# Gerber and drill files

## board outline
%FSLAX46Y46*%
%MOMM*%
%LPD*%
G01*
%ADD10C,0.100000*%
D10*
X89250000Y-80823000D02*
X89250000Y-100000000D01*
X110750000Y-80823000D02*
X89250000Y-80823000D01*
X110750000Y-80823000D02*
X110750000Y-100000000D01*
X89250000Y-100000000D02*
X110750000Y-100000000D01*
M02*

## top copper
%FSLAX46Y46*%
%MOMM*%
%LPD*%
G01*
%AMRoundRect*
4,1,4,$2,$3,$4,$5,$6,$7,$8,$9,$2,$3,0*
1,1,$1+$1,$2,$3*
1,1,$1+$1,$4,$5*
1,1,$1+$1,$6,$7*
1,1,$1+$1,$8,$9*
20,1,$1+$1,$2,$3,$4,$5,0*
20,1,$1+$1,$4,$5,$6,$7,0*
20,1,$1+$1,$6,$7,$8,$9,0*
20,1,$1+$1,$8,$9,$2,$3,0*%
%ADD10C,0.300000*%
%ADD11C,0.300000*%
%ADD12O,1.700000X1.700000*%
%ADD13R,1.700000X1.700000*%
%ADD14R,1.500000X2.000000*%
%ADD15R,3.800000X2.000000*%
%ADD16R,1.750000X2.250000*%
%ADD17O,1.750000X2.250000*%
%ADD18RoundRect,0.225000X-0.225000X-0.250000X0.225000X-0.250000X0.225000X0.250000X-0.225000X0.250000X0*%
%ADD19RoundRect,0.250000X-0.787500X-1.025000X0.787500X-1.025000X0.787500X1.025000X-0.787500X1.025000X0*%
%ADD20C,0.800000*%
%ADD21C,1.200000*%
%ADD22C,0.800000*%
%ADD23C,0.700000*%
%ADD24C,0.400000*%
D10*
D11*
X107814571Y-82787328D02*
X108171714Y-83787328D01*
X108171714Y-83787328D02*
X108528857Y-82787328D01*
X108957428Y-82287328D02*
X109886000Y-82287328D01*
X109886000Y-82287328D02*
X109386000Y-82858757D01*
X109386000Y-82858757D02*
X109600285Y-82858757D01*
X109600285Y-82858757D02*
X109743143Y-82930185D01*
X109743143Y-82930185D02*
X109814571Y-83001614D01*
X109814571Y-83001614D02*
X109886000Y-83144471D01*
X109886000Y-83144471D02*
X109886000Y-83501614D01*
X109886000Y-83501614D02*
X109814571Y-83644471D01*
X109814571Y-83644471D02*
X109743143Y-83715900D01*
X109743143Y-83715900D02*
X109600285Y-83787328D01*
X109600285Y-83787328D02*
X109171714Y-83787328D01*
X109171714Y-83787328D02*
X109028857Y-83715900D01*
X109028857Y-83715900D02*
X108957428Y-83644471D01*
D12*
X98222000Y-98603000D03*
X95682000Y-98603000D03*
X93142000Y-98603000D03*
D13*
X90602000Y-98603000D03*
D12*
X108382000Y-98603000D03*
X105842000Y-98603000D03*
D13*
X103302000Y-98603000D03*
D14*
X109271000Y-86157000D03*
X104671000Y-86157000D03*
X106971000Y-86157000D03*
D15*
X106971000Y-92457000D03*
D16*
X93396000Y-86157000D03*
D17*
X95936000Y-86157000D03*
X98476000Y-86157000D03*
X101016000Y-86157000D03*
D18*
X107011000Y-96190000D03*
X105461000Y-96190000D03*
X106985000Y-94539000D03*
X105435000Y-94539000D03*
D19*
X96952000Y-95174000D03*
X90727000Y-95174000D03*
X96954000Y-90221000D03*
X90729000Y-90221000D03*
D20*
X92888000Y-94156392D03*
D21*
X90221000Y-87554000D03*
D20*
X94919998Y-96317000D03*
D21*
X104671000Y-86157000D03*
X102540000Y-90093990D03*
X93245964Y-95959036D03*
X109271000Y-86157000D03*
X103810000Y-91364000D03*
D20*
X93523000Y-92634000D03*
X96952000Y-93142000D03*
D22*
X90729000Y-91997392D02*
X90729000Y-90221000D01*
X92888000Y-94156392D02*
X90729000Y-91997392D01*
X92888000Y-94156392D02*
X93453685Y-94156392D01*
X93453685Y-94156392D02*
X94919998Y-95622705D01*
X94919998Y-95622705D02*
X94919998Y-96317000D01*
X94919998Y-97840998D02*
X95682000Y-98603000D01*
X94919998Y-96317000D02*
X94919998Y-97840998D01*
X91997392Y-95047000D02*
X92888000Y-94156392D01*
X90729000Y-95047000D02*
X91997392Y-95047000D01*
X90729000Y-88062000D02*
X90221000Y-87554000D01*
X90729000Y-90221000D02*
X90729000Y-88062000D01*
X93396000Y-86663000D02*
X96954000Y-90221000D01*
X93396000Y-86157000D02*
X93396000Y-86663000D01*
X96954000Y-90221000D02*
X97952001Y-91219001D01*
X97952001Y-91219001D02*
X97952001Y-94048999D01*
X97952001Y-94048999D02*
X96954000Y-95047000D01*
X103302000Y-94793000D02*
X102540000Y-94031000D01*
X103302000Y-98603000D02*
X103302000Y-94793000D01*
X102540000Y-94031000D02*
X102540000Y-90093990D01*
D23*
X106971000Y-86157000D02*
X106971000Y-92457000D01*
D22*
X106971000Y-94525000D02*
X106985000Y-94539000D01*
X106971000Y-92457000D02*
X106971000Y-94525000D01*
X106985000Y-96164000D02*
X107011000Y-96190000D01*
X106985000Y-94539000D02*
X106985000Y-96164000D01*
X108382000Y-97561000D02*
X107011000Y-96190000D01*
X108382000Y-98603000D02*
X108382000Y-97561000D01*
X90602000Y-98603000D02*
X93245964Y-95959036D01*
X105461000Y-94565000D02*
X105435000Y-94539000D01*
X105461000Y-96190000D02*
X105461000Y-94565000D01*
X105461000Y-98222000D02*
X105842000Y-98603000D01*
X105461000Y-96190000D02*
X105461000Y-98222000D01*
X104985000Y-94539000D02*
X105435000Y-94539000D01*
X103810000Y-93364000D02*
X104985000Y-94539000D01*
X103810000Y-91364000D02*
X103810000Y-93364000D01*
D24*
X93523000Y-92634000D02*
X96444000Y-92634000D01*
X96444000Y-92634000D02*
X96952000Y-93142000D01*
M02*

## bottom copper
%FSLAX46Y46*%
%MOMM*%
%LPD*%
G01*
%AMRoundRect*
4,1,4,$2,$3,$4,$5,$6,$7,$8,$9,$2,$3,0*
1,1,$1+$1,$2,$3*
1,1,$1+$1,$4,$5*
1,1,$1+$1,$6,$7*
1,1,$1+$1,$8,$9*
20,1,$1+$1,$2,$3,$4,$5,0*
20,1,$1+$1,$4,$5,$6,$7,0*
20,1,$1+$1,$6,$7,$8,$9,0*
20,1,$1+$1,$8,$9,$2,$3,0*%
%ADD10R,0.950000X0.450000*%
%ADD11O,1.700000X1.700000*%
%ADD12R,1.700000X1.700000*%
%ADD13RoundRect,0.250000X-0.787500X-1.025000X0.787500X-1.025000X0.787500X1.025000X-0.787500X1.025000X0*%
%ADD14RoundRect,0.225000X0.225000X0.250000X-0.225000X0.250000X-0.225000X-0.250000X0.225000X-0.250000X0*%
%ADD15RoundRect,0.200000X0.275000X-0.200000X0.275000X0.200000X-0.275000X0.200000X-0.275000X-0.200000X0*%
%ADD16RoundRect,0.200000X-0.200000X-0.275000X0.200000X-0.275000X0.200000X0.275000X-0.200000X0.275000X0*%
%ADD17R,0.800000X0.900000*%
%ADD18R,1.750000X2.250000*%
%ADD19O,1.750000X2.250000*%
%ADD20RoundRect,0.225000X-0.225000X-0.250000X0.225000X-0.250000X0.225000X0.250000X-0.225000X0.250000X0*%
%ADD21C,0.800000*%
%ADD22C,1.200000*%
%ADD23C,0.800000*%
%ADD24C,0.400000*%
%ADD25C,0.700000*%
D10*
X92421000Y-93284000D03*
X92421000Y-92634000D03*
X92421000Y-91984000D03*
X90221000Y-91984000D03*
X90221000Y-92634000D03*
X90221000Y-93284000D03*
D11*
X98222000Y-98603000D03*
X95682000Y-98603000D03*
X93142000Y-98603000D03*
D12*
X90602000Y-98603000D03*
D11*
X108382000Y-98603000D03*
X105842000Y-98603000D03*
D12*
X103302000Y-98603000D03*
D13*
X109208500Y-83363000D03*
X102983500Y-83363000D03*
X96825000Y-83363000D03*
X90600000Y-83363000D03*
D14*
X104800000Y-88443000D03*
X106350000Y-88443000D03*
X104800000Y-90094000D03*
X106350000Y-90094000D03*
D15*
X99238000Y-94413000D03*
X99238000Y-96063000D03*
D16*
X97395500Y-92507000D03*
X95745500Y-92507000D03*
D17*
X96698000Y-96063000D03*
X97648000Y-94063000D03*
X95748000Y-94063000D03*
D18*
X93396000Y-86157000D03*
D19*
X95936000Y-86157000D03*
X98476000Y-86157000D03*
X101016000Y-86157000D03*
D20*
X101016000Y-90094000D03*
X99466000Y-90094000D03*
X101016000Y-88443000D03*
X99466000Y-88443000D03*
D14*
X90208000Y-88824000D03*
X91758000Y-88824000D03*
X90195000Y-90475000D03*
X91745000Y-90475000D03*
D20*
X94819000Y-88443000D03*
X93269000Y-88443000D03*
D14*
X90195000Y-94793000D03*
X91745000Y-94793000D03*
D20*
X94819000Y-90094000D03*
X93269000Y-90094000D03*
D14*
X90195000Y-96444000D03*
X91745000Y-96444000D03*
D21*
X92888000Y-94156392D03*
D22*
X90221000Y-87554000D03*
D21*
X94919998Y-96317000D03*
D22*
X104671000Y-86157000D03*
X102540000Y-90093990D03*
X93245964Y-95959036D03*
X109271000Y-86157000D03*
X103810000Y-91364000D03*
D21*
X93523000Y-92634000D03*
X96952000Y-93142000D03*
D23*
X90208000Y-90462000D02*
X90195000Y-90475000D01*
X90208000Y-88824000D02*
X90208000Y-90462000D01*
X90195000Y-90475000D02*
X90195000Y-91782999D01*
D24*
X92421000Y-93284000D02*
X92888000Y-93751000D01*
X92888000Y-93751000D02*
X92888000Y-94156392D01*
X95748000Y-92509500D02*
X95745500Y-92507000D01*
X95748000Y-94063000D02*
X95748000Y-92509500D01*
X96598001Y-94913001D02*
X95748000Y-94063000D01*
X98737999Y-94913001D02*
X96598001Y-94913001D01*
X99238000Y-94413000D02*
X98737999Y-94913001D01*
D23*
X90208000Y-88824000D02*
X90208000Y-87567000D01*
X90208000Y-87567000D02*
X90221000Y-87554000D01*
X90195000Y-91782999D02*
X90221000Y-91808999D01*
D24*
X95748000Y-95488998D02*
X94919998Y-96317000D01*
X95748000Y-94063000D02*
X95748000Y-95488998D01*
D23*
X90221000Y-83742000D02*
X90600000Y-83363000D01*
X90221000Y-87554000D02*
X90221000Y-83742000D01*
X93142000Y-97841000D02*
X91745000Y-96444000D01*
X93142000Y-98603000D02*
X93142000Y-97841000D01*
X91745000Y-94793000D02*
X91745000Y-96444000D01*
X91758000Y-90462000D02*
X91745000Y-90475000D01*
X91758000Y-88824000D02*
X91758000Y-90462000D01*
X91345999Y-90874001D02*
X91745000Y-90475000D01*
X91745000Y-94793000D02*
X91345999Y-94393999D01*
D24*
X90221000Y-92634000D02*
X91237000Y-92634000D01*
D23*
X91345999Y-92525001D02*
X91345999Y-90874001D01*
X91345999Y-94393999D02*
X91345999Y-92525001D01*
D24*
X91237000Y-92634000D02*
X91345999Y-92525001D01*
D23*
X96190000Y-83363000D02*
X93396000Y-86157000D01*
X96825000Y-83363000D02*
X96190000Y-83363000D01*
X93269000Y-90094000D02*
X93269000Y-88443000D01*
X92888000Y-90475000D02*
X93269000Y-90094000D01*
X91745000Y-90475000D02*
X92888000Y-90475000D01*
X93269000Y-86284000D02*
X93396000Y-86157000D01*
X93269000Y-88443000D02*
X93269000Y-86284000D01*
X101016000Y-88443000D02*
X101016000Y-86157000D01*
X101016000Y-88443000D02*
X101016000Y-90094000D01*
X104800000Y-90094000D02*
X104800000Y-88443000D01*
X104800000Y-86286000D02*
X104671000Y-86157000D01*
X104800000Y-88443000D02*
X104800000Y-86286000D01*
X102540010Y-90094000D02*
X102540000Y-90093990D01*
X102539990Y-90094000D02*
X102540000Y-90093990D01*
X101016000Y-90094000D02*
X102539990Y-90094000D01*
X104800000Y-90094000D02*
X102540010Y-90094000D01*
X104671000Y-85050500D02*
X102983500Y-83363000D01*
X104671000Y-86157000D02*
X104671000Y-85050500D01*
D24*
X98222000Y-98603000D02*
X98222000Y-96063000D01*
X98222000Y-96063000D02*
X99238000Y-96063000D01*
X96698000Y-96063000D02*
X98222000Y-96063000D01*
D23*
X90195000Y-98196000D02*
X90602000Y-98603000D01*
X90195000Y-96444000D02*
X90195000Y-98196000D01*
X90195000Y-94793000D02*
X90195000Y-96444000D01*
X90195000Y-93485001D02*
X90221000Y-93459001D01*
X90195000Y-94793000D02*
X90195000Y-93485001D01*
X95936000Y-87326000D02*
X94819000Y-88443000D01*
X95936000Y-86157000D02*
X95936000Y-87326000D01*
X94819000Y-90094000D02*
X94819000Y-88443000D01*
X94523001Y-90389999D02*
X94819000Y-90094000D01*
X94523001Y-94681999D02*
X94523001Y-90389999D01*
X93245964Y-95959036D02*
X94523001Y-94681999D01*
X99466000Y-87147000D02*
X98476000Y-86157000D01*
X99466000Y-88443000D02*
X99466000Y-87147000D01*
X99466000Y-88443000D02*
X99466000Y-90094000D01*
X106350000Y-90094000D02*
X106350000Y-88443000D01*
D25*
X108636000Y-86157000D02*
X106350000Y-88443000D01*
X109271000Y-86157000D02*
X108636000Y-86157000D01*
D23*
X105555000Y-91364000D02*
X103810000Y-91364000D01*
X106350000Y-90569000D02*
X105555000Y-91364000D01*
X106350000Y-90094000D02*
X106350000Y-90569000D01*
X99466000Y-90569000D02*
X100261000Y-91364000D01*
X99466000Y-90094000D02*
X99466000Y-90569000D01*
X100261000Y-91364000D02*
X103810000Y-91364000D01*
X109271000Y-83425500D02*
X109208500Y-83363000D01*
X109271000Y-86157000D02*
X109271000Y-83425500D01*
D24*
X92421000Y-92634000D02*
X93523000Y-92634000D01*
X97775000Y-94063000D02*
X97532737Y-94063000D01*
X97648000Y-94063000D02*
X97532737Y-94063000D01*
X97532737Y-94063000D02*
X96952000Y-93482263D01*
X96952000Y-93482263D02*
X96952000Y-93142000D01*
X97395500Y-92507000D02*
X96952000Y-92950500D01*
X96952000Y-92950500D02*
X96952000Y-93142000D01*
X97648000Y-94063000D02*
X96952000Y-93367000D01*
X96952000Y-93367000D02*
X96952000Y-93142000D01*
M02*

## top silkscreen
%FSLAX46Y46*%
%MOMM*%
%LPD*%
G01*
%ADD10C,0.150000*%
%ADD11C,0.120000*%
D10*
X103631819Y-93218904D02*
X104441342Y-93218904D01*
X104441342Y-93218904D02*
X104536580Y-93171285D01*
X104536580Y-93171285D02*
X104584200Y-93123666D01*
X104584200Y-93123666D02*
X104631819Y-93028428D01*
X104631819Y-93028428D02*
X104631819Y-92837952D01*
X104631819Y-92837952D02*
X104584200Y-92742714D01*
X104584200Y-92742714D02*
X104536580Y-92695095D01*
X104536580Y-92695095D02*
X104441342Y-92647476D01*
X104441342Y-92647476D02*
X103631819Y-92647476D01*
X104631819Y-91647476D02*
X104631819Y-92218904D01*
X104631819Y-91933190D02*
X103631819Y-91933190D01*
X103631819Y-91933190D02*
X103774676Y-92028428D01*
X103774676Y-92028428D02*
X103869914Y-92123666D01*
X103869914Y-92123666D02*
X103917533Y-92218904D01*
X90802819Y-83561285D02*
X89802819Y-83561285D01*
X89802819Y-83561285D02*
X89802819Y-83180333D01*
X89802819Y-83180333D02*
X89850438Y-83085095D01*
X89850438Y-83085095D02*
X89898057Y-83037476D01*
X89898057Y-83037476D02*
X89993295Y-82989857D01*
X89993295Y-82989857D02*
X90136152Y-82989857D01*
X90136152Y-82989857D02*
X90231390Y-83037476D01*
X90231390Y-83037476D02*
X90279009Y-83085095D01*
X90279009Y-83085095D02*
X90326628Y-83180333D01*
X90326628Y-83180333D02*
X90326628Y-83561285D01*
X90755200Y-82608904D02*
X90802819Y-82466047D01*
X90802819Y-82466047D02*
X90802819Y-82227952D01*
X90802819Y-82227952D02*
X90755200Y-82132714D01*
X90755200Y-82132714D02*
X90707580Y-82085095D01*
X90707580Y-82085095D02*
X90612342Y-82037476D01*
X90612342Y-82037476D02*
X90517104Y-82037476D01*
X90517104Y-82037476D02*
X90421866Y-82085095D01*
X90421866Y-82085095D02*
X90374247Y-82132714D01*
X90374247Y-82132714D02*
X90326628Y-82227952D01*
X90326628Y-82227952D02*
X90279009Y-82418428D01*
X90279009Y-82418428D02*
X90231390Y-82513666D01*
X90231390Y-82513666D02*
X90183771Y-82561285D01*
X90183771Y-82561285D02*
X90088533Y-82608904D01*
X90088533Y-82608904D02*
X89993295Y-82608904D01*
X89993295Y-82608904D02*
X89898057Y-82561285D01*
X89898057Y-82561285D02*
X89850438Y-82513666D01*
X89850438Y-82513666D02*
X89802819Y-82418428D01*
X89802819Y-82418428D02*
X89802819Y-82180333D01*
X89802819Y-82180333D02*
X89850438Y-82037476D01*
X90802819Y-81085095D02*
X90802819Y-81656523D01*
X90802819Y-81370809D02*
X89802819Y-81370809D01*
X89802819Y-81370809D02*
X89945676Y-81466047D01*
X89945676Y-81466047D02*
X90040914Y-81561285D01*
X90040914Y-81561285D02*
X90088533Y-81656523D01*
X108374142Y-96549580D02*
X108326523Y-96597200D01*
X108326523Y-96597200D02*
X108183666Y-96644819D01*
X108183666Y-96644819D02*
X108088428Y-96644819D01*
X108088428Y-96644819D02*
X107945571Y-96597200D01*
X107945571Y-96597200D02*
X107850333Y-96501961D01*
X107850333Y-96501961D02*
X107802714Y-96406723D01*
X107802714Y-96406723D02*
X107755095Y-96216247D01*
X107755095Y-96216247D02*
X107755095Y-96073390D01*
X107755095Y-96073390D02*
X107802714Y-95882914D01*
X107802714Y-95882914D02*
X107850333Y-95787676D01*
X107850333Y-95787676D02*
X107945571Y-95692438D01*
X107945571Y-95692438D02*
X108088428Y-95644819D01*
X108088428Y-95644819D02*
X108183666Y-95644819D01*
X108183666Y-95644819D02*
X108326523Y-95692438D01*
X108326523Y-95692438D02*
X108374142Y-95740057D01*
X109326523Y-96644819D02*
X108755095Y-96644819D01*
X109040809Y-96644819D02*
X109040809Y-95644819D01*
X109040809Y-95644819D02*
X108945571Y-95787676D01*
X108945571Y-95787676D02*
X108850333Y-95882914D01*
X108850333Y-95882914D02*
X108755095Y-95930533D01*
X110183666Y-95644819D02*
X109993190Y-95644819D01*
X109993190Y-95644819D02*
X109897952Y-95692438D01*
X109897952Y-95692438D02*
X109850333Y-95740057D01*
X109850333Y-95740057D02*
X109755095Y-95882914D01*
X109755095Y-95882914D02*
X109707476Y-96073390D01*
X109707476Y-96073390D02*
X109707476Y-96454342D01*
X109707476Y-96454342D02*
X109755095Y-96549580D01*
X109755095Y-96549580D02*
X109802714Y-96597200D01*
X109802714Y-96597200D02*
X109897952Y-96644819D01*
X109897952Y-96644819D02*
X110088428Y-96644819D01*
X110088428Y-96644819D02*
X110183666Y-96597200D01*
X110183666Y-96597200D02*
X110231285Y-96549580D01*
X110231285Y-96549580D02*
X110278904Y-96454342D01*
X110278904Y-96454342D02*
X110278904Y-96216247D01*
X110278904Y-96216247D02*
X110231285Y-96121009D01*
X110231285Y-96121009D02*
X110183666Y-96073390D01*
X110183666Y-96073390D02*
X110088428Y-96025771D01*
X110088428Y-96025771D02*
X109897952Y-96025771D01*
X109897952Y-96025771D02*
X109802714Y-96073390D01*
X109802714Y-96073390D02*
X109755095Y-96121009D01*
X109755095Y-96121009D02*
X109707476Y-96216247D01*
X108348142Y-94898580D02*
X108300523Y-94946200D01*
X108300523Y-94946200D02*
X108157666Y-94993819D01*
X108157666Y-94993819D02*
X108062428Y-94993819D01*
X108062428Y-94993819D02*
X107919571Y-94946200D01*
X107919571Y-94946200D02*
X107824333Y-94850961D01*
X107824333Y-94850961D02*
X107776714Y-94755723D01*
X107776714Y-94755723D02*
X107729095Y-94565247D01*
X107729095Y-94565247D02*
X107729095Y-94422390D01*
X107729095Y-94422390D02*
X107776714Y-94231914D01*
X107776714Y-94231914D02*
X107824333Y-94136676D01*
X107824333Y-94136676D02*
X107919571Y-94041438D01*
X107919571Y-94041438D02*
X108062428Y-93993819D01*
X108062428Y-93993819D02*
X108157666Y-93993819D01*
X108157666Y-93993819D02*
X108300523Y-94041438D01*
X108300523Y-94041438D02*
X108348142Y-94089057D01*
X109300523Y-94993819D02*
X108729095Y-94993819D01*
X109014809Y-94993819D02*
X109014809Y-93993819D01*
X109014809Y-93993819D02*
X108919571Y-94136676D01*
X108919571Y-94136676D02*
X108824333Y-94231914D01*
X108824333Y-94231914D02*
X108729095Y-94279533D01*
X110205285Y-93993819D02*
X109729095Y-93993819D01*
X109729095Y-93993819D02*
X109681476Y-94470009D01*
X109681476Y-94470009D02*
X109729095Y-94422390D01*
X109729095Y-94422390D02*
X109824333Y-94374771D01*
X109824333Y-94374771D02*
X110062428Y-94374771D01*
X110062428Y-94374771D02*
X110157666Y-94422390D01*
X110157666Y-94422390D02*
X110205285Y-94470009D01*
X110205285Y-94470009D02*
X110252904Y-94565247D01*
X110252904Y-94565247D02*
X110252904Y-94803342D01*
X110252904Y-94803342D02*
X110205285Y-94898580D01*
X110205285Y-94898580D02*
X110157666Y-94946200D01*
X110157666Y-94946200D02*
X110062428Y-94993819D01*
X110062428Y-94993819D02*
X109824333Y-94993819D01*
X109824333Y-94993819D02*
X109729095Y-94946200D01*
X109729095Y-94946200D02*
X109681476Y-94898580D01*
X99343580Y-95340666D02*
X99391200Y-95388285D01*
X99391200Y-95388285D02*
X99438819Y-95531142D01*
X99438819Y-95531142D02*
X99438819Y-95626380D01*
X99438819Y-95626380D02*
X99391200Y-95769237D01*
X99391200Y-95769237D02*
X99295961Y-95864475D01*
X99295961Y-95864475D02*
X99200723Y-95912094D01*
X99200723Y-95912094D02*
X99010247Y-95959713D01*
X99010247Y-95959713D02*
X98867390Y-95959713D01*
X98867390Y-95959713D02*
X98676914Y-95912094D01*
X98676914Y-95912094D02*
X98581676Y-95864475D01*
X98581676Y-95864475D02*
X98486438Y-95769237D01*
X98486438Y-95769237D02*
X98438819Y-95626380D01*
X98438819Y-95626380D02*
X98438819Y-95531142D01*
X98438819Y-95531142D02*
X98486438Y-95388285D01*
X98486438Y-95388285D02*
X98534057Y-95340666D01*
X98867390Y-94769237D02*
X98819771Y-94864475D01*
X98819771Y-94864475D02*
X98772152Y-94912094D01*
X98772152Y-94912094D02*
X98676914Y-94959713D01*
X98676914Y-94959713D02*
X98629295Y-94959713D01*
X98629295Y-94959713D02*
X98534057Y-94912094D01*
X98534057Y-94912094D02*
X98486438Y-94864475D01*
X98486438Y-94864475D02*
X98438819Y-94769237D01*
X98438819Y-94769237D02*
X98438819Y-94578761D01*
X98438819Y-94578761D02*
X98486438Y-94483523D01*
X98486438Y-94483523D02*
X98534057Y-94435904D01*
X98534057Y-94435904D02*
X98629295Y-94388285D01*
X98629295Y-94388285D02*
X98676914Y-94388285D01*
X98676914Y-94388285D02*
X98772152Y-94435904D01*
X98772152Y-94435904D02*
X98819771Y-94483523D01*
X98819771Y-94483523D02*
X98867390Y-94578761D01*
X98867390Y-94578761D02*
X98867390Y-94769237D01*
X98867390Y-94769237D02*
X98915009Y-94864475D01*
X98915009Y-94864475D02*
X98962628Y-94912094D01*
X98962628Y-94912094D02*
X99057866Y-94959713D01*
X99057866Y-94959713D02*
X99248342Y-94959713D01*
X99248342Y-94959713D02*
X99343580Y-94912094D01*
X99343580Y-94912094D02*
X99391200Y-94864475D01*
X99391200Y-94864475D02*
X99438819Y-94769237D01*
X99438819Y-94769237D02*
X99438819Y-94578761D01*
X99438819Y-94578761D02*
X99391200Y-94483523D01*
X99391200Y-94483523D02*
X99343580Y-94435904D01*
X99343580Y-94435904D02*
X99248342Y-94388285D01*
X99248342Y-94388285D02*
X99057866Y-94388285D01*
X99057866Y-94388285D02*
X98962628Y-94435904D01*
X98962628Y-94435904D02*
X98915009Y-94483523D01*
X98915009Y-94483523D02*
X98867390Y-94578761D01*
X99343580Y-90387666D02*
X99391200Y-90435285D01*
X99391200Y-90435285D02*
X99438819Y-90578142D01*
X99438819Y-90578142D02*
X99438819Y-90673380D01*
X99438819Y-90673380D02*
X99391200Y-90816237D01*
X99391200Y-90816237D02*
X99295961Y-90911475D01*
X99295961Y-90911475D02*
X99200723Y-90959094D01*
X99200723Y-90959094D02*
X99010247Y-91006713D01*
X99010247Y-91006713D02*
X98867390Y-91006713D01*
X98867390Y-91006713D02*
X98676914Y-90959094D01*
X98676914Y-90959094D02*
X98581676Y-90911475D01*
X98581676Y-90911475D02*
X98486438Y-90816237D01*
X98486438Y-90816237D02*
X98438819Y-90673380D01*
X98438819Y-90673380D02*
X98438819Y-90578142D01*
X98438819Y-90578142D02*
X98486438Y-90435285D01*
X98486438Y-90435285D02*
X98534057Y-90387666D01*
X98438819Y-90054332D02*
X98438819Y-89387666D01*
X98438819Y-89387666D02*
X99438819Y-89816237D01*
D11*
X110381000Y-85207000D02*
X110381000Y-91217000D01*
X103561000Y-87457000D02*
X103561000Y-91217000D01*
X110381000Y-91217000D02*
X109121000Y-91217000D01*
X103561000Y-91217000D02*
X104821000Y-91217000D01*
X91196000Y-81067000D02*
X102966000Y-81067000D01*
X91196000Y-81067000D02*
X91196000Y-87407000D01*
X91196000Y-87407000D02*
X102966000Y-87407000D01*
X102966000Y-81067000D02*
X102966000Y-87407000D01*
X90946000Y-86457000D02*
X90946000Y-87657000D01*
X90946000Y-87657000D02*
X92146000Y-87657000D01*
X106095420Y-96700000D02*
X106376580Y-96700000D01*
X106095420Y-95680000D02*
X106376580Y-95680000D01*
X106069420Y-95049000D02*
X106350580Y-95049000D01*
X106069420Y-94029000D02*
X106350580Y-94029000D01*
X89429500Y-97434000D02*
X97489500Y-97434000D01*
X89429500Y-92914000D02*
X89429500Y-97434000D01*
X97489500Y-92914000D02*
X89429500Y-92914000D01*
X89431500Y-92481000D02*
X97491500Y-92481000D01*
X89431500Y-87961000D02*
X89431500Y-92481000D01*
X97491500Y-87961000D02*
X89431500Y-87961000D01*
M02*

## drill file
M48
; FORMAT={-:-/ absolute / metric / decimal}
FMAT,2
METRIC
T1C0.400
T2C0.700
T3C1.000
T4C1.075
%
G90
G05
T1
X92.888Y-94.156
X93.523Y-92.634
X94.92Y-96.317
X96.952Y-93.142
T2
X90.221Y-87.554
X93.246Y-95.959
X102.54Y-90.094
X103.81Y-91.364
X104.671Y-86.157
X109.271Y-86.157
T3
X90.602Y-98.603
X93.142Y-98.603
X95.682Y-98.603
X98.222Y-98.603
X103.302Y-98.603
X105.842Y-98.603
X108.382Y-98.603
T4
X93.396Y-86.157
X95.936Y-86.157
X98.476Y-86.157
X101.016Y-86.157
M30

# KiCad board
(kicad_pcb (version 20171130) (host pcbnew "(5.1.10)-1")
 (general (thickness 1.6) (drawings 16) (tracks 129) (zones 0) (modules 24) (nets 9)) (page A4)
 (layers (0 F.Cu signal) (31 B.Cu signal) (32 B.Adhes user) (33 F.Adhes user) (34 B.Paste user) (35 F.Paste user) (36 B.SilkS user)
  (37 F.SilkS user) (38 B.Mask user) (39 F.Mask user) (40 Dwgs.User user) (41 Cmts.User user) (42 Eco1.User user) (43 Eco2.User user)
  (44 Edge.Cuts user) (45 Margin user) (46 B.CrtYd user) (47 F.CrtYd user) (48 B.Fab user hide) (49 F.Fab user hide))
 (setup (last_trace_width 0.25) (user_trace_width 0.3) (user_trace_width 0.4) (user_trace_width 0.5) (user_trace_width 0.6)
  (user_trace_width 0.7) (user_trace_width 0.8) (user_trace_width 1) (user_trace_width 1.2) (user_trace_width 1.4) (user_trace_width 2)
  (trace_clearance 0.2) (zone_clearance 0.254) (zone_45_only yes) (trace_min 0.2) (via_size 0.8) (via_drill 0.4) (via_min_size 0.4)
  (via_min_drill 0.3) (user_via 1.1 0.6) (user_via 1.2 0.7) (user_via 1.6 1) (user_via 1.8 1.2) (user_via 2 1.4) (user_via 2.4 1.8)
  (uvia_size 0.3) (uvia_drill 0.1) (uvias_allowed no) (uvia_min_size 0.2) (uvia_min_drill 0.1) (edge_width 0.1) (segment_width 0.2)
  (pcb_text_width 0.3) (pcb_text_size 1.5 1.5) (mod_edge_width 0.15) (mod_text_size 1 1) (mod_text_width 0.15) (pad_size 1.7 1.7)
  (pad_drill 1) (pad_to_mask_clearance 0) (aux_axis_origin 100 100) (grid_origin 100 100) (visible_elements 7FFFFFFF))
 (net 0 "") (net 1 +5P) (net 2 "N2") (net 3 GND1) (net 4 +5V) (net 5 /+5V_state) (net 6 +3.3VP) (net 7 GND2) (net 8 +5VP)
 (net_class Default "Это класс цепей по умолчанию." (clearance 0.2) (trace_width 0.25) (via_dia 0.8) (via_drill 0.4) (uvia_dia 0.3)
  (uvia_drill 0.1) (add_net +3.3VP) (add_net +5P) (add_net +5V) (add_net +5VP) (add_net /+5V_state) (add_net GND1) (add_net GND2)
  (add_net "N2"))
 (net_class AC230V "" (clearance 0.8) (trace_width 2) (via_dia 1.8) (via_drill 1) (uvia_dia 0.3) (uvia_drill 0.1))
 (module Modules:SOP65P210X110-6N (layer B.Cu) (at 91.321 92.634)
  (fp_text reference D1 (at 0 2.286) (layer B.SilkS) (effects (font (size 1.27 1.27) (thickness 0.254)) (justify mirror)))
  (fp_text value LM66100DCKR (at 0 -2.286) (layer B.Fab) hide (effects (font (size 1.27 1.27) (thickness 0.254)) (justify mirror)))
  (pad 6 smd rect (at 1.1 0.65 270) (size 0.45 0.95) (layers B.Cu B.Paste B.Mask) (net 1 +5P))
  (pad 5 smd rect (at 1.1 0 270) (size 0.45 0.95) (layers B.Cu B.Paste B.Mask) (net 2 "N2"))
  (pad 4 smd rect (at 1.1 -0.65 270) (size 0.45 0.95) (layers B.Cu B.Paste B.Mask))
  (pad 3 smd rect (at -1.1 -0.65 270) (size 0.45 0.95) (layers B.Cu B.Paste B.Mask) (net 1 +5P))
  (pad 2 smd rect (at -1.1 0 270) (size 0.45 0.95) (layers B.Cu B.Paste B.Mask) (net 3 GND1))
  (pad 1 smd rect (at -1.1 0.65 270) (size 0.45 0.95) (layers B.Cu B.Paste B.Mask) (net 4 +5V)))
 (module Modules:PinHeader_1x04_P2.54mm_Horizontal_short (layer B.Cu) (at 90.602 98.603 270)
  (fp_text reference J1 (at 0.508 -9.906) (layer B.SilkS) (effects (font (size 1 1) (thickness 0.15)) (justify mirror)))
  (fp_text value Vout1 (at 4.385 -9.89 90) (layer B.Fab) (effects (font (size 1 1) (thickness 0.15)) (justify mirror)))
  (pad 4 thru_hole oval (at 0 -7.62 270) (size 1.7 1.7) (drill 1) (layers *.Cu *.Mask) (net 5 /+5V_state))
  (pad 3 thru_hole oval (at 0 -5.08 270) (size 1.7 1.7) (drill 1) (layers *.Cu *.Mask) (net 1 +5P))
  (pad 2 thru_hole oval (at 0 -2.54 270) (size 1.7 1.7) (drill 1) (layers *.Cu *.Mask) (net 3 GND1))
  (pad 1 thru_hole rect (at 0 0 270) (size 1.7 1.7) (drill 1) (layers *.Cu *.Mask) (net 4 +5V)))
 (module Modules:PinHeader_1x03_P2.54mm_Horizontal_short (layer B.Cu) (at 103.302 98.603 270)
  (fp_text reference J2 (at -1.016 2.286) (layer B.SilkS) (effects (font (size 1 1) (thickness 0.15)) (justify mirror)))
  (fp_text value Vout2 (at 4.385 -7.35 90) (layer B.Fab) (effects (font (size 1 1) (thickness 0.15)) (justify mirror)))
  (pad 3 thru_hole oval (at 0 -5.08 270) (size 1.7 1.7) (drill 1) (layers *.Cu *.Mask) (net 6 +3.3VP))
  (pad 2 thru_hole oval (at 0 -2.54 270) (size 1.7 1.7) (drill 1) (layers *.Cu *.Mask) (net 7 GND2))
  (pad 1 thru_hole rect (at 0 0 270) (size 1.7 1.7) (drill 1) (layers *.Cu *.Mask) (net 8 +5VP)))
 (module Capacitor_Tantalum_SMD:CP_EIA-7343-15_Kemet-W (layer B.Cu) (at 106.096 83.363)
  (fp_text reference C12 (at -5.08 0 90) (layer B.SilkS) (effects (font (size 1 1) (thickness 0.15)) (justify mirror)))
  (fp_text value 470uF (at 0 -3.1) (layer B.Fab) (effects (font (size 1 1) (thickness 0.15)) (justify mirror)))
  (pad 2 smd roundrect (at 3.1125 0) (size 2.075 2.55) (layers B.Cu B.Paste B.Mask) (roundrect_rratio 0.1204819277108434) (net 7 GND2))
  (pad 1 smd roundrect (at -3.1125 0) (size 2.075 2.55) (layers B.Cu B.Paste B.Mask) (roundrect_rratio 0.1204819277108434) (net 8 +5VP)))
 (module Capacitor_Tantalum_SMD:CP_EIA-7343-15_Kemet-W (layer B.Cu) (at 93.7125 83.363)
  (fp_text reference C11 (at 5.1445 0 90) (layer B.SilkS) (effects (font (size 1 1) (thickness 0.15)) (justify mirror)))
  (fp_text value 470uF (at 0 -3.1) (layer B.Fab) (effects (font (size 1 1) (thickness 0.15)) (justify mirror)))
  (pad 2 smd roundrect (at 3.1125 0) (size 2.075 2.55) (layers B.Cu B.Paste B.Mask) (roundrect_rratio 0.1204819277108434) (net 3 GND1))
  (pad 1 smd roundrect (at -3.1125 0) (size 2.075 2.55) (layers B.Cu B.Paste B.Mask) (roundrect_rratio 0.1204819277108434) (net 1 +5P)))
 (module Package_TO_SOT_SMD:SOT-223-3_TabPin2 (layer F.Cu) (at 106.971 89.307 270)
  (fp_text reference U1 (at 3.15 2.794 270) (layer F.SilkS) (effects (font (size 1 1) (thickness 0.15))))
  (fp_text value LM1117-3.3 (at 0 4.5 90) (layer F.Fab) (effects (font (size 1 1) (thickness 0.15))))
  (fp_line (start -4.1 -3.41) (end 1.91 -3.41) (layer F.SilkS) (width 0.12))
  (fp_line (start -1.85 3.41) (end 1.91 3.41) (layer F.SilkS) (width 0.12))
  (fp_line (start 1.91 -3.41) (end 1.91 -2.15) (layer F.SilkS) (width 0.12))
  (fp_line (start 1.91 3.41) (end 1.91 2.15) (layer F.SilkS) (width 0.12))
  (pad 1 smd rect (at -3.15 -2.3 270) (size 2 1.5) (layers F.Cu F.Paste F.Mask) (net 7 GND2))
  (pad 3 smd rect (at -3.15 2.3 270) (size 2 1.5) (layers F.Cu F.Paste F.Mask) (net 8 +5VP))
  (pad 2 smd rect (at -3.15 0 270) (size 2 1.5) (layers F.Cu F.Paste F.Mask) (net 6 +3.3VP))
  (pad 2 smd rect (at 3.15 0 270) (size 2 3.8) (layers F.Cu F.Paste F.Mask) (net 6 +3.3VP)))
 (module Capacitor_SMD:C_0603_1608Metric (layer B.Cu) (at 105.575 88.443 180)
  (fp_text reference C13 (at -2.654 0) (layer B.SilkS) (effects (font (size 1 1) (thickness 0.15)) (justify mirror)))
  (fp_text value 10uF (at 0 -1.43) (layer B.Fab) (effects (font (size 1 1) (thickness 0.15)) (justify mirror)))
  (pad 2 smd roundrect (at 0.775 0 180) (size 0.9 0.95) (layers B.Cu B.Paste B.Mask) (roundrect_rratio 0.25) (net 8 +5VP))
  (pad 1 smd roundrect (at -0.775 0 180) (size 0.9 0.95) (layers B.Cu B.Paste B.Mask) (roundrect_rratio 0.25) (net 7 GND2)))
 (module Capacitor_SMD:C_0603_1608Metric (layer B.Cu) (at 105.575 90.094 180)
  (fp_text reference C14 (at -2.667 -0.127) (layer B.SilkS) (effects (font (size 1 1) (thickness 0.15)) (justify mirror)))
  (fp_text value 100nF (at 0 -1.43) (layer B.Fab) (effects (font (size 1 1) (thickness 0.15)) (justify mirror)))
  (pad 2 smd roundrect (at 0.775 0 180) (size 0.9 0.95) (layers B.Cu B.Paste B.Mask) (roundrect_rratio 0.25) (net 8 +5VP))
  (pad 1 smd roundrect (at -0.775 0 180) (size 0.9 0.95) (layers B.Cu B.Paste B.Mask) (roundrect_rratio 0.25) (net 7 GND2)))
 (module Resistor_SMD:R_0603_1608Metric (layer B.Cu) (at 99.238 95.238 90)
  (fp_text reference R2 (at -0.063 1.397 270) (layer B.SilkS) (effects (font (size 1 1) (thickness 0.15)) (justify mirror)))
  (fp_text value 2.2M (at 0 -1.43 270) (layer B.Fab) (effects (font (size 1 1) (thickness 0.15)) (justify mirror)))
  (pad 2 smd roundrect (at 0.825 0 90) (size 0.8 0.95) (layers B.Cu B.Paste B.Mask) (roundrect_rratio 0.25) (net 1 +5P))
  (pad 1 smd roundrect (at -0.825 0 90) (size 0.8 0.95) (layers B.Cu B.Paste B.Mask) (roundrect_rratio 0.25) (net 5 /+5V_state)))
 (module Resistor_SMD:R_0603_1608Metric (layer B.Cu) (at 96.5705 92.507)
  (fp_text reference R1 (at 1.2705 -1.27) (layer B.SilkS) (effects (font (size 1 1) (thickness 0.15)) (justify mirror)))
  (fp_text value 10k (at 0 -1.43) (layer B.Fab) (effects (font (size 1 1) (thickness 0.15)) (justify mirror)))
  (pad 2 smd roundrect (at 0.825 0) (size 0.8 0.95) (layers B.Cu B.Paste B.Mask) (roundrect_rratio 0.25) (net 2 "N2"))
  (pad 1 smd roundrect (at -0.825 0) (size 0.8 0.95) (layers B.Cu B.Paste B.Mask) (roundrect_rratio 0.25) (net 1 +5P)))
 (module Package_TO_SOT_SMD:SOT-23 (layer B.Cu) (at 96.698 95.063 270)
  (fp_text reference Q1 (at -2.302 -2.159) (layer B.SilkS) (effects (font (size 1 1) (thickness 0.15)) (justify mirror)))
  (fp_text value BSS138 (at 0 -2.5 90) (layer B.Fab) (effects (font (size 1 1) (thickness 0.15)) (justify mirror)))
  (pad 3 smd rect (at 1 0 270) (size 0.9 0.8) (layers B.Cu B.Paste B.Mask) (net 5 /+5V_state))
  (pad 2 smd rect (at -1 -0.95 270) (size 0.9 0.8) (layers B.Cu B.Paste B.Mask) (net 2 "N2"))
  (pad 1 smd rect (at -1 0.95 270) (size 0.9 0.8) (layers B.Cu B.Paste B.Mask) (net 1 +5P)))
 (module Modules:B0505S (layer F.Cu) (at 93.396 86.157 90)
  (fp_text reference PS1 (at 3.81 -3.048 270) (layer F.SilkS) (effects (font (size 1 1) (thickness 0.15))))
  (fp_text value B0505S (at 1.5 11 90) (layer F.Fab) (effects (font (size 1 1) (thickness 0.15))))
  (fp_line (start 5.09 -2.2) (end 5.09 9.57) (layer F.SilkS) (width 0.12))
  (fp_line (start 5.09 -2.2) (end -1.25 -2.2) (layer F.SilkS) (width 0.12))
  (fp_line (start -1.25 -2.2) (end -1.25 9.57) (layer F.SilkS) (width 0.12))
  (fp_line (start 5.09 9.57) (end -1.25 9.57) (layer F.SilkS) (width 0.12))
  (fp_line (start -0.3 -2.45) (end -1.5 -2.45) (layer F.SilkS) (width 0.12))
  (fp_line (start -1.5 -2.45) (end -1.5 -1.25) (layer F.SilkS) (width 0.12))
  (pad 1 thru_hole rect (at 0 0) (size 1.75 2.25) (drill 1.075) (layers *.Cu *.Mask) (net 3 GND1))
  (pad 2 thru_hole oval (at 0 2.54) (size 1.75 2.25) (drill 1.075) (layers *.Cu *.Mask) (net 4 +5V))
  (pad 3 thru_hole oval (at 0 5.08) (size 1.75 2.25) (drill 1.075) (layers *.Cu *.Mask) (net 7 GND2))
  (pad 4 thru_hole oval (at 0 7.62) (size 1.75 2.25) (drill 1.075) (layers *.Cu *.Mask) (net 8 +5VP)))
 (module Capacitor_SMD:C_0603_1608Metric (layer F.Cu) (at 106.236 96.19)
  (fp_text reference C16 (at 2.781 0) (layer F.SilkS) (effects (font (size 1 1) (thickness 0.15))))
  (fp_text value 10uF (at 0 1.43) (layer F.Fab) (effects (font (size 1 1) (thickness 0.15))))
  (fp_line (start -0.14058 0.51) (end 0.14058 0.51) (layer F.SilkS) (width 0.12))
  (fp_line (start -0.14058 -0.51) (end 0.14058 -0.51) (layer F.SilkS) (width 0.12))
  (pad 2 smd roundrect (at 0.775 0) (size 0.9 0.95) (layers F.Cu F.Paste F.Mask) (roundrect_rratio 0.25) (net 6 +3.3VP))
  (pad 1 smd roundrect (at -0.775 0) (size 0.9 0.95) (layers F.Cu F.Paste F.Mask) (roundrect_rratio 0.25) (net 7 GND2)))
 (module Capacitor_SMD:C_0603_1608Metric (layer F.Cu) (at 106.21 94.539)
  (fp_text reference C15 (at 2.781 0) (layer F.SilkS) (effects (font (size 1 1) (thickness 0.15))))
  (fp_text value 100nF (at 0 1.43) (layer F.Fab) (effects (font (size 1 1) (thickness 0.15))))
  (fp_line (start -0.14058 0.51) (end 0.14058 0.51) (layer F.SilkS) (width 0.12))
  (fp_line (start -0.14058 -0.51) (end 0.14058 -0.51) (layer F.SilkS) (width 0.12))
  (pad 2 smd roundrect (at 0.775 0) (size 0.9 0.95) (layers F.Cu F.Paste F.Mask) (roundrect_rratio 0.25) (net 6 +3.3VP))
  (pad 1 smd roundrect (at -0.775 0) (size 0.9 0.95) (layers F.Cu F.Paste F.Mask) (roundrect_rratio 0.25) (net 7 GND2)))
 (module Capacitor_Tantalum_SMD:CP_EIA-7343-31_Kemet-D (layer F.Cu) (at 93.8395 95.174)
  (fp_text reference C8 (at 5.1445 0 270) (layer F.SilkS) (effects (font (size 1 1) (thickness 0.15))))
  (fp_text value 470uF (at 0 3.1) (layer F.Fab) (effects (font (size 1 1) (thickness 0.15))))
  (fp_line (start -4.41 2.26) (end 3.65 2.26) (layer F.SilkS) (width 0.12))
  (fp_line (start -4.41 -2.26) (end -4.41 2.26) (layer F.SilkS) (width 0.12))
  (fp_line (start 3.65 -2.26) (end -4.41 -2.26) (layer F.SilkS) (width 0.12))
  (pad 2 smd roundrect (at 3.1125 0) (size 2.075 2.55) (layers F.Cu F.Paste F.Mask) (roundrect_rratio 0.1204819277108434) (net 3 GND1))
  (pad 1 smd roundrect (at -3.1125 0) (size 2.075 2.55) (layers F.Cu F.Paste F.Mask) (roundrect_rratio 0.1204819277108434) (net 1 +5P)))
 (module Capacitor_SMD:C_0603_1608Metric (layer B.Cu) (at 100.241 90.094)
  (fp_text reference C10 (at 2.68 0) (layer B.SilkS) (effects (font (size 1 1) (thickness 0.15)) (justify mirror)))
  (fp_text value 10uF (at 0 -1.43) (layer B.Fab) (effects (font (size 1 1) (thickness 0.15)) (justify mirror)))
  (pad 2 smd roundrect (at 0.775 0) (size 0.9 0.95) (layers B.Cu B.Paste B.Mask) (roundrect_rratio 0.25) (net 8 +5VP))
  (pad 1 smd roundrect (at -0.775 0) (size 0.9 0.95) (layers B.Cu B.Paste B.Mask) (roundrect_rratio 0.25) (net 7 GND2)))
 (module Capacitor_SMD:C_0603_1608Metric (layer B.Cu) (at 100.241 88.443)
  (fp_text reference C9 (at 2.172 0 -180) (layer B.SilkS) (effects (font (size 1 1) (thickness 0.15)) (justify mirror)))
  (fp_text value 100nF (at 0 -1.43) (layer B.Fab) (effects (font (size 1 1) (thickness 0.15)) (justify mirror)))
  (pad 2 smd roundrect (at 0.775 0) (size 0.9 0.95) (layers B.Cu B.Paste B.Mask) (roundrect_rratio 0.25) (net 8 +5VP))
  (pad 1 smd roundrect (at -0.775 0) (size 0.9 0.95) (layers B.Cu B.Paste B.Mask) (roundrect_rratio 0.25) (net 7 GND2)))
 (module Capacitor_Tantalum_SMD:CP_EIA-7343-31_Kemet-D (layer F.Cu) (at 93.8415 90.221)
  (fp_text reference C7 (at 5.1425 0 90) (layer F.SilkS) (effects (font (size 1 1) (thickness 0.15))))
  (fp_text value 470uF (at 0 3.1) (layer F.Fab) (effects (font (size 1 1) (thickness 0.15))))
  (fp_line (start -4.41 2.26) (end 3.65 2.26) (layer F.SilkS) (width 0.12))
  (fp_line (start -4.41 -2.26) (end -4.41 2.26) (layer F.SilkS) (width 0.12))
  (fp_line (start 3.65 -2.26) (end -4.41 -2.26) (layer F.SilkS) (width 0.12))
  (pad 2 smd roundrect (at 3.1125 0) (size 2.075 2.55) (layers F.Cu F.Paste F.Mask) (roundrect_rratio 0.1204819277108434) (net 3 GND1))
  (pad 1 smd roundrect (at -3.1125 0) (size 2.075 2.55) (layers F.Cu F.Paste F.Mask) (roundrect_rratio 0.1204819277108434) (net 1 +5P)))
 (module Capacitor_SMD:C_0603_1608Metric (layer B.Cu) (at 90.983 88.824 180)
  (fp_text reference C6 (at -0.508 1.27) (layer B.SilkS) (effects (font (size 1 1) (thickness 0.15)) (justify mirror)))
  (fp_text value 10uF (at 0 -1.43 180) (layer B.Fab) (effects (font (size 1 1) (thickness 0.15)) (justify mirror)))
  (pad 2 smd roundrect (at 0.775 0 180) (size 0.9 0.95) (layers B.Cu B.Paste B.Mask) (roundrect_rratio 0.25) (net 1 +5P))
  (pad 1 smd roundrect (at -0.775 0 180) (size 0.9 0.95) (layers B.Cu B.Paste B.Mask) (roundrect_rratio 0.25) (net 3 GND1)))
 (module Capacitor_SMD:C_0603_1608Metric (layer B.Cu) (at 90.97 90.475 180)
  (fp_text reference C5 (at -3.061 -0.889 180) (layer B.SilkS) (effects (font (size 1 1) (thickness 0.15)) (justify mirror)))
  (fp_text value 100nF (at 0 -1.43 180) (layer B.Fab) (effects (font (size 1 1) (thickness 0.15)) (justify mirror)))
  (pad 2 smd roundrect (at 0.775 0 180) (size 0.9 0.95) (layers B.Cu B.Paste B.Mask) (roundrect_rratio 0.25) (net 1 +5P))
  (pad 1 smd roundrect (at -0.775 0 180) (size 0.9 0.95) (layers B.Cu B.Paste B.Mask) (roundrect_rratio 0.25) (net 3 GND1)))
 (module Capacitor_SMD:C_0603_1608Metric (layer B.Cu) (at 94.044 88.443)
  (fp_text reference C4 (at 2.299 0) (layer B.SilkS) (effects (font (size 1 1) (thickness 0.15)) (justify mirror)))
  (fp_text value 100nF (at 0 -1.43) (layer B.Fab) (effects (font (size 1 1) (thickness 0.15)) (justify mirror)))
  (pad 2 smd roundrect (at 0.775 0) (size 0.9 0.95) (layers B.Cu B.Paste B.Mask) (roundrect_rratio 0.25) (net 4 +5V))
  (pad 1 smd roundrect (at -0.775 0) (size 0.9 0.95) (layers B.Cu B.Paste B.Mask) (roundrect_rratio 0.25) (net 3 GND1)))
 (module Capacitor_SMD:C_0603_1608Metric (layer B.Cu) (at 90.97 94.793 180)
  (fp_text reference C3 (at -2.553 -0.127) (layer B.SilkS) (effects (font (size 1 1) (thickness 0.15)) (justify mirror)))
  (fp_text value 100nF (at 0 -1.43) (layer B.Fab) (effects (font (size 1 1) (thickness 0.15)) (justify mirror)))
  (pad 2 smd roundrect (at 0.775 0 180) (size 0.9 0.95) (layers B.Cu B.Paste B.Mask) (roundrect_rratio 0.25) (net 4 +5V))
  (pad 1 smd roundrect (at -0.775 0 180) (size 0.9 0.95) (layers B.Cu B.Paste B.Mask) (roundrect_rratio 0.25) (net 3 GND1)))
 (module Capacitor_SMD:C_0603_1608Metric (layer B.Cu) (at 94.044 90.094)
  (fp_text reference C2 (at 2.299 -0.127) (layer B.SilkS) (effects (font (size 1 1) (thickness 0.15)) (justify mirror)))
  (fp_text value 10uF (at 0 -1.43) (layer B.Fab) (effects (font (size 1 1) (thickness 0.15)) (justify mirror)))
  (pad 2 smd roundrect (at 0.775 0) (size 0.9 0.95) (layers B.Cu B.Paste B.Mask) (roundrect_rratio 0.25) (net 4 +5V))
  (pad 1 smd roundrect (at -0.775 0) (size 0.9 0.95) (layers B.Cu B.Paste B.Mask) (roundrect_rratio 0.25) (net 3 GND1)))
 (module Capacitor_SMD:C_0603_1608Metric (layer B.Cu) (at 90.97 96.444 180)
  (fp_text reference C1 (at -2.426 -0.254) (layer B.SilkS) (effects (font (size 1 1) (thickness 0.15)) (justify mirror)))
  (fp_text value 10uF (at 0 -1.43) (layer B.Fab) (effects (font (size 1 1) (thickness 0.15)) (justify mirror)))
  (pad 2 smd roundrect (at 0.775 0 180) (size 0.9 0.95) (layers B.Cu B.Paste B.Mask) (roundrect_rratio 0.25) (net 4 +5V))
  (pad 1 smd roundrect (at -0.775 0 180) (size 0.9 0.95) (layers B.Cu B.Paste B.Mask) (roundrect_rratio 0.25) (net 3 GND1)))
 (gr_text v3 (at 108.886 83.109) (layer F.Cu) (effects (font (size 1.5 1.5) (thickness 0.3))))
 (gr_line (start 89.25 80.823) (end 89.25 100) (layer Edge.Cuts) (width 0.1))
 (gr_line (start 110.75 80.823) (end 89.25 80.823) (layer Edge.Cuts) (width 0.1))
 (gr_line (start 110.75 80.823) (end 110.75 100) (layer Edge.Cuts) (width 0.1))
 (gr_line (start 89.25 100) (end 110.75 100) (layer Edge.Cuts) (width 0.1))
 (segment (start 90.208 90.462) (end 90.195 90.475) (width 0.8) (layer B.Cu) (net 1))
 (segment (start 90.208 88.824) (end 90.208 90.462) (width 0.8) (layer B.Cu) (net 1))
 (segment (start 90.195 90.475) (end 90.195 91.782999) (width 0.8) (layer B.Cu) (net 1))
 (via (at 92.888 94.156392) (size 0.8) (drill 0.4) (layers F.Cu B.Cu) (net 1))
 (segment (start 92.421 93.284) (end 92.888 93.751) (width 0.4) (layer B.Cu) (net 1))
 (segment (start 92.888 93.751) (end 92.888 94.156392) (width 0.4) (layer B.Cu) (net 1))
 (segment (start 95.748 92.5095) (end 95.7455 92.507) (width 0.4) (layer B.Cu) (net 1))
 (segment (start 95.748 94.063) (end 95.748 92.5095) (width 0.4) (layer B.Cu) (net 1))
 (segment (start 96.598001 94.913001) (end 95.748 94.063) (width 0.4) (layer B.Cu) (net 1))
 (segment (start 98.737999 94.913001) (end 96.598001 94.913001) (width 0.4) (layer B.Cu) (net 1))
 (segment (start 99.238 94.413) (end 98.737999 94.913001) (width 0.4) (layer B.Cu) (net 1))
 (via (at 90.221 87.554) (size 1.2) (drill 0.7) (layers F.Cu B.Cu) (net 1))
 (segment (start 90.208 88.824) (end 90.208 87.567) (width 0.8) (layer B.Cu) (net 1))
 (segment (start 90.208 87.567) (end 90.221 87.554) (width 0.8) (layer B.Cu) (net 1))
 (segment (start 90.195 91.782999) (end 90.221 91.808999) (width 0.8) (layer B.Cu) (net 1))
 (segment (start 90.729 91.997392) (end 90.729 90.221) (width 0.8) (layer F.Cu) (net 1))
 (segment (start 92.888 94.156392) (end 90.729 91.997392) (width 0.8) (layer F.Cu) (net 1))
 (segment (start 92.888 94.156392) (end 93.453685 94.156392) (width 0.8) (layer F.Cu) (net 1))
 (segment (start 95.748 95.488998) (end 94.919998 96.317) (width 0.4) (layer B.Cu) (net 1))
 (segment (start 93.453685 94.156392) (end 94.919998 95.622705) (width 0.8) (layer F.Cu) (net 1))
 (segment (start 95.748 94.063) (end 95.748 95.488998) (width 0.4) (layer B.Cu) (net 1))
 (via (at 94.919998 96.317) (size 0.8) (drill 0.4) (layers F.Cu B.Cu) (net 1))
 (segment (start 94.919998 95.622705) (end 94.919998 96.317) (width 0.8) (layer F.Cu) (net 1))
 (segment (start 94.919998 97.840998) (end 95.682 98.603) (width 0.8) (layer F.Cu) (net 1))
 (segment (start 94.919998 96.317) (end 94.919998 97.840998) (width 0.8) (layer F.Cu) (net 1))
 (segment (start 91.997392 95.047) (end 92.888 94.156392) (width 0.8) (layer F.Cu) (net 1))
 (segment (start 90.729 95.047) (end 91.997392 95.047) (width 0.8) (layer F.Cu) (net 1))
 (segment (start 90.729 88.062) (end 90.221 87.554) (width 0.8) (layer F.Cu) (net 1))
 (segment (start 90.729 90.221) (end 90.729 88.062) (width 0.8) (layer F.Cu) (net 1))
 (segment (start 90.221 83.742) (end 90.6 83.363) (width 0.8) (layer B.Cu) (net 1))
 (segment (start 90.221 87.554) (end 90.221 83.742) (width 0.8) (layer B.Cu) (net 1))
 (segment (start 93.142 97.841) (end 91.745 96.444) (width 0.8) (layer B.Cu) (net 3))
 (segment (start 93.142 98.603) (end 93.142 97.841) (width 0.8) (layer B.Cu) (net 3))
 (segment (start 91.745 94.793) (end 91.745 96.444) (width 0.8) (layer B.Cu) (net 3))
 (segment (start 91.758 90.462) (end 91.745 90.475) (width 0.8) (layer B.Cu) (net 3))
 (segment (start 91.758 88.824) (end 91.758 90.462) (width 0.8) (layer B.Cu) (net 3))
 (segment (start 91.345999 90.874001) (end 91.745 90.475) (width 0.8) (layer B.Cu) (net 3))
 (segment (start 91.745 94.793) (end 91.345999 94.393999) (width 0.8) (layer B.Cu) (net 3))
 (segment (start 90.221 92.634) (end 91.237 92.634) (width 0.4) (layer B.Cu) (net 3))
 (segment (start 91.345999 92.525001) (end 91.345999 90.874001) (width 0.8) (layer B.Cu) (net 3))
 (segment (start 91.345999 94.393999) (end 91.345999 92.525001) (width 0.8) (layer B.Cu) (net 3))
 (segment (start 91.237 92.634) (end 91.345999 92.525001) (width 0.4) (layer B.Cu) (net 3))
 (segment (start 93.396 86.663) (end 96.954 90.221) (width 0.8) (layer F.Cu) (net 3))
 (segment (start 93.396 86.157) (end 93.396 86.663) (width 0.8) (layer F.Cu) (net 3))
 (segment (start 96.19 83.363) (end 93.396 86.157) (width 0.8) (layer B.Cu) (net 3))
 (segment (start 96.825 83.363) (end 96.19 83.363) (width 0.8) (layer B.Cu) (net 3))
 (segment (start 96.954 90.221) (end 97.952001 91.219001) (width 0.8) (layer F.Cu) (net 3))
 (segment (start 97.952001 91.219001) (end 97.952001 94.048999) (width 0.8) (layer F.Cu) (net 3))
 (segment (start 97.952001 94.048999) (end 96.954 95.047) (width 0.8) (layer F.Cu) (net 3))
 (segment (start 93.269 90.094) (end 93.269 88.443) (width 0.8) (layer B.Cu) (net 3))
 (segment (start 92.888 90.475) (end 93.269 90.094) (width 0.8) (layer B.Cu) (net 3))
 (segment (start 91.745 90.475) (end 92.888 90.475) (width 0.8) (layer B.Cu) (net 3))
 (segment (start 93.269 86.284) (end 93.396 86.157) (width 0.8) (layer B.Cu) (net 3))
 (segment (start 93.269 88.443) (end 93.269 86.284) (width 0.8) (layer B.Cu) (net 3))
 (segment (start 101.016 88.443) (end 101.016 86.157) (width 0.8) (layer B.Cu) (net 8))
 (segment (start 101.016 88.443) (end 101.016 90.094) (width 0.8) (layer B.Cu) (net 8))
 (segment (start 104.8 90.094) (end 104.8 88.443) (width 0.8) (layer B.Cu) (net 8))
 (via (at 104.671 86.157) (size 1.2) (drill 0.7) (layers F.Cu B.Cu) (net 8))
 (segment (start 104.8 86.286) (end 104.671 86.157) (width 0.8) (layer B.Cu) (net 8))
 (segment (start 104.8 88.443) (end 104.8 86.286) (width 0.8) (layer B.Cu) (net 8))
 (segment (start 102.54001 90.094) (end 102.54 90.09399) (width 0.8) (layer B.Cu) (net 8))
 (segment (start 102.53999 90.094) (end 102.54 90.09399) (width 0.8) (layer B.Cu) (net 8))
 (segment (start 101.016 90.094) (end 102.53999 90.094) (width 0.8) (layer B.Cu) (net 8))
 (segment (start 104.8 90.094) (end 102.54001 90.094) (width 0.8) (layer B.Cu) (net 8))
 (via (at 102.54 90.09399) (size 1.2) (drill 0.7) (layers F.Cu B.Cu) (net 8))
 (segment (start 103.302 94.793) (end 102.54 94.031) (width 0.8) (layer F.Cu) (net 8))
 (segment (start 103.302 98.603) (end 103.302 94.793) (width 0.8) (layer F.Cu) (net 8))
 (segment (start 102.54 94.031) (end 102.54 90.09399) (width 0.8) (layer F.Cu) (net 8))
 (segment (start 104.671 85.0505) (end 102.9835 83.363) (width 0.8) (layer B.Cu) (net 8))
 (segment (start 104.671 86.157) (end 104.671 85.0505) (width 0.8) (layer B.Cu) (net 8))
 (segment (start 98.222 98.603) (end 98.222 96.063) (width 0.4) (layer B.Cu) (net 5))
 (segment (start 98.222 96.063) (end 99.238 96.063) (width 0.4) (layer B.Cu) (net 5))
 (segment (start 96.698 96.063) (end 98.222 96.063) (width 0.4) (layer B.Cu) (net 5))
 (segment (start 106.971 86.157) (end 106.971 92.457) (width 0.7) (layer F.Cu) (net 6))
 (segment (start 106.971 94.525) (end 106.985 94.539) (width 0.8) (layer F.Cu) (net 6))
 (segment (start 106.971 92.457) (end 106.971 94.525) (width 0.8) (layer F.Cu) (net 6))
 (segment (start 106.985 96.164) (end 107.011 96.19) (width 0.8) (layer F.Cu) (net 6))
 (segment (start 106.985 94.539) (end 106.985 96.164) (width 0.8) (layer F.Cu) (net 6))
 (segment (start 108.382 97.561) (end 107.011 96.19) (width 0.8) (layer F.Cu) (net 6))
 (segment (start 108.382 98.603) (end 108.382 97.561) (width 0.8) (layer F.Cu) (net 6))
 (segment (start 90.195 98.196) (end 90.602 98.603) (width 0.8) (layer B.Cu) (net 4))
 (segment (start 90.195 96.444) (end 90.195 98.196) (width 0.8) (layer B.Cu) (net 4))
 (segment (start 90.195 94.793) (end 90.195 96.444) (width 0.8) (layer B.Cu) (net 4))
 (segment (start 90.195 93.485001) (end 90.221 93.459001) (width 0.8) (layer B.Cu) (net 4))
 (segment (start 90.195 94.793) (end 90.195 93.485001) (width 0.8) (layer B.Cu) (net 4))
 (segment (start 90.602 98.603) (end 93.245964 95.959036) (width 0.8) (layer F.Cu) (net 4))
 (via (at 93.245964 95.959036) (size 1.2) (drill 0.7) (layers F.Cu B.Cu) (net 4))
 (segment (start 95.936 87.326) (end 94.819 88.443) (width 0.8) (layer B.Cu) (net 4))
 (segment (start 95.936 86.157) (end 95.936 87.326) (width 0.8) (layer B.Cu) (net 4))
 (segment (start 94.819 90.094) (end 94.819 88.443) (width 0.8) (layer B.Cu) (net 4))
 (segment (start 94.523001 90.389999) (end 94.819 90.094) (width 0.8) (layer B.Cu) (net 4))
 (segment (start 94.523001 94.681999) (end 94.523001 90.389999) (width 0.8) (layer B.Cu) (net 4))
 (segment (start 93.245964 95.959036) (end 94.523001 94.681999) (width 0.8) (layer B.Cu) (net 4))
 (segment (start 99.466 87.147) (end 98.476 86.157) (width 0.8) (layer B.Cu) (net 7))
 (segment (start 99.466 88.443) (end 99.466 87.147) (width 0.8) (layer B.Cu) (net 7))
 (segment (start 99.466 88.443) (end 99.466 90.094) (width 0.8) (layer B.Cu) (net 7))
 (segment (start 106.35 90.094) (end 106.35 88.443) (width 0.8) (layer B.Cu) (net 7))
 (via (at 109.271 86.157) (size 1.2) (drill 0.7) (layers F.Cu B.Cu) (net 7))
 (segment (start 108.636 86.157) (end 106.35 88.443) (width 0.7) (layer B.Cu) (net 7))
 (segment (start 109.271 86.157) (end 108.636 86.157) (width 0.7) (layer B.Cu) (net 7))
 (segment (start 105.555 91.364) (end 103.81 91.364) (width 0.8) (layer B.Cu) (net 7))
 (segment (start 106.35 90.569) (end 105.555 91.364) (width 0.8) (layer B.Cu) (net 7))
 (segment (start 106.35 90.094) (end 106.35 90.569) (width 0.8) (layer B.Cu) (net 7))
 (segment (start 99.466 90.569) (end 100.261 91.364) (width 0.8) (layer B.Cu) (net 7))
 (segment (start 99.466 90.094) (end 99.466 90.569) (width 0.8) (layer B.Cu) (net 7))
 (segment (start 100.261 91.364) (end 103.81 91.364) (width 0.8) (layer B.Cu) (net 7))
 (via (at 103.81 91.364) (size 1.2) (drill 0.7) (layers F.Cu B.Cu) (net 7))
 (segment (start 105.461 94.565) (end 105.435 94.539) (width 0.8) (layer F.Cu) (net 7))
 (segment (start 105.461 96.19) (end 105.461 94.565) (width 0.8) (layer F.Cu) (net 7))
 (segment (start 105.461 98.222) (end 105.842 98.603) (width 0.8) (layer F.Cu) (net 7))
 (segment (start 105.461 96.19) (end 105.461 98.222) (width 0.8) (layer F.Cu) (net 7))
 (segment (start 104.985 94.539) (end 105.435 94.539) (width 0.8) (layer F.Cu) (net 7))
 (segment (start 103.81 93.364) (end 104.985 94.539) (width 0.8) (layer F.Cu) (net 7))
 (segment (start 103.81 91.364) (end 103.81 93.364) (width 0.8) (layer F.Cu) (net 7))
 (segment (start 109.271 83.4255) (end 109.2085 83.363) (width 0.8) (layer B.Cu) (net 7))
 (segment (start 109.271 86.157) (end 109.271 83.4255) (width 0.8) (layer B.Cu) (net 7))
 (via (at 93.523 92.634) (size 0.8) (drill 0.4) (layers F.Cu B.Cu) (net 2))
 (segment (start 92.421 92.634) (end 93.523 92.634) (width 0.4) (layer B.Cu) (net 2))
 (segment (start 97.775 94.063) (end 97.532737 94.063) (width 0.4) (layer B.Cu) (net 2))
 (segment (start 97.648 94.063) (end 97.532737 94.063) (width 0.4) (layer B.Cu) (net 2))
 (segment (start 97.532737 94.063) (end 96.952 93.482263) (width 0.4) (layer B.Cu) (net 2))
 (segment (start 96.952 93.482263) (end 96.952 93.142) (width 0.4) (layer B.Cu) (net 2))
 (segment (start 97.3955 92.507) (end 96.952 92.9505) (width 0.4) (layer B.Cu) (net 2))
 (segment (start 96.952 92.9505) (end 96.952 93.142) (width 0.4) (layer B.Cu) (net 2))
 (segment (start 97.648 94.063) (end 96.952 93.367) (width 0.4) (layer B.Cu) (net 2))
 (segment (start 96.952 93.367) (end 96.952 93.142) (width 0.4) (layer B.Cu) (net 2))
 (segment (start 93.523 92.634) (end 96.444 92.634) (width 0.4) (layer F.Cu) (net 2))
 (segment (start 96.444 92.634) (end 96.952 93.142) (width 0.4) (layer F.Cu) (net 2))
 (via (at 96.952 93.142) (size 0.8) (drill 0.4) (layers F.Cu B.Cu) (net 2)))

